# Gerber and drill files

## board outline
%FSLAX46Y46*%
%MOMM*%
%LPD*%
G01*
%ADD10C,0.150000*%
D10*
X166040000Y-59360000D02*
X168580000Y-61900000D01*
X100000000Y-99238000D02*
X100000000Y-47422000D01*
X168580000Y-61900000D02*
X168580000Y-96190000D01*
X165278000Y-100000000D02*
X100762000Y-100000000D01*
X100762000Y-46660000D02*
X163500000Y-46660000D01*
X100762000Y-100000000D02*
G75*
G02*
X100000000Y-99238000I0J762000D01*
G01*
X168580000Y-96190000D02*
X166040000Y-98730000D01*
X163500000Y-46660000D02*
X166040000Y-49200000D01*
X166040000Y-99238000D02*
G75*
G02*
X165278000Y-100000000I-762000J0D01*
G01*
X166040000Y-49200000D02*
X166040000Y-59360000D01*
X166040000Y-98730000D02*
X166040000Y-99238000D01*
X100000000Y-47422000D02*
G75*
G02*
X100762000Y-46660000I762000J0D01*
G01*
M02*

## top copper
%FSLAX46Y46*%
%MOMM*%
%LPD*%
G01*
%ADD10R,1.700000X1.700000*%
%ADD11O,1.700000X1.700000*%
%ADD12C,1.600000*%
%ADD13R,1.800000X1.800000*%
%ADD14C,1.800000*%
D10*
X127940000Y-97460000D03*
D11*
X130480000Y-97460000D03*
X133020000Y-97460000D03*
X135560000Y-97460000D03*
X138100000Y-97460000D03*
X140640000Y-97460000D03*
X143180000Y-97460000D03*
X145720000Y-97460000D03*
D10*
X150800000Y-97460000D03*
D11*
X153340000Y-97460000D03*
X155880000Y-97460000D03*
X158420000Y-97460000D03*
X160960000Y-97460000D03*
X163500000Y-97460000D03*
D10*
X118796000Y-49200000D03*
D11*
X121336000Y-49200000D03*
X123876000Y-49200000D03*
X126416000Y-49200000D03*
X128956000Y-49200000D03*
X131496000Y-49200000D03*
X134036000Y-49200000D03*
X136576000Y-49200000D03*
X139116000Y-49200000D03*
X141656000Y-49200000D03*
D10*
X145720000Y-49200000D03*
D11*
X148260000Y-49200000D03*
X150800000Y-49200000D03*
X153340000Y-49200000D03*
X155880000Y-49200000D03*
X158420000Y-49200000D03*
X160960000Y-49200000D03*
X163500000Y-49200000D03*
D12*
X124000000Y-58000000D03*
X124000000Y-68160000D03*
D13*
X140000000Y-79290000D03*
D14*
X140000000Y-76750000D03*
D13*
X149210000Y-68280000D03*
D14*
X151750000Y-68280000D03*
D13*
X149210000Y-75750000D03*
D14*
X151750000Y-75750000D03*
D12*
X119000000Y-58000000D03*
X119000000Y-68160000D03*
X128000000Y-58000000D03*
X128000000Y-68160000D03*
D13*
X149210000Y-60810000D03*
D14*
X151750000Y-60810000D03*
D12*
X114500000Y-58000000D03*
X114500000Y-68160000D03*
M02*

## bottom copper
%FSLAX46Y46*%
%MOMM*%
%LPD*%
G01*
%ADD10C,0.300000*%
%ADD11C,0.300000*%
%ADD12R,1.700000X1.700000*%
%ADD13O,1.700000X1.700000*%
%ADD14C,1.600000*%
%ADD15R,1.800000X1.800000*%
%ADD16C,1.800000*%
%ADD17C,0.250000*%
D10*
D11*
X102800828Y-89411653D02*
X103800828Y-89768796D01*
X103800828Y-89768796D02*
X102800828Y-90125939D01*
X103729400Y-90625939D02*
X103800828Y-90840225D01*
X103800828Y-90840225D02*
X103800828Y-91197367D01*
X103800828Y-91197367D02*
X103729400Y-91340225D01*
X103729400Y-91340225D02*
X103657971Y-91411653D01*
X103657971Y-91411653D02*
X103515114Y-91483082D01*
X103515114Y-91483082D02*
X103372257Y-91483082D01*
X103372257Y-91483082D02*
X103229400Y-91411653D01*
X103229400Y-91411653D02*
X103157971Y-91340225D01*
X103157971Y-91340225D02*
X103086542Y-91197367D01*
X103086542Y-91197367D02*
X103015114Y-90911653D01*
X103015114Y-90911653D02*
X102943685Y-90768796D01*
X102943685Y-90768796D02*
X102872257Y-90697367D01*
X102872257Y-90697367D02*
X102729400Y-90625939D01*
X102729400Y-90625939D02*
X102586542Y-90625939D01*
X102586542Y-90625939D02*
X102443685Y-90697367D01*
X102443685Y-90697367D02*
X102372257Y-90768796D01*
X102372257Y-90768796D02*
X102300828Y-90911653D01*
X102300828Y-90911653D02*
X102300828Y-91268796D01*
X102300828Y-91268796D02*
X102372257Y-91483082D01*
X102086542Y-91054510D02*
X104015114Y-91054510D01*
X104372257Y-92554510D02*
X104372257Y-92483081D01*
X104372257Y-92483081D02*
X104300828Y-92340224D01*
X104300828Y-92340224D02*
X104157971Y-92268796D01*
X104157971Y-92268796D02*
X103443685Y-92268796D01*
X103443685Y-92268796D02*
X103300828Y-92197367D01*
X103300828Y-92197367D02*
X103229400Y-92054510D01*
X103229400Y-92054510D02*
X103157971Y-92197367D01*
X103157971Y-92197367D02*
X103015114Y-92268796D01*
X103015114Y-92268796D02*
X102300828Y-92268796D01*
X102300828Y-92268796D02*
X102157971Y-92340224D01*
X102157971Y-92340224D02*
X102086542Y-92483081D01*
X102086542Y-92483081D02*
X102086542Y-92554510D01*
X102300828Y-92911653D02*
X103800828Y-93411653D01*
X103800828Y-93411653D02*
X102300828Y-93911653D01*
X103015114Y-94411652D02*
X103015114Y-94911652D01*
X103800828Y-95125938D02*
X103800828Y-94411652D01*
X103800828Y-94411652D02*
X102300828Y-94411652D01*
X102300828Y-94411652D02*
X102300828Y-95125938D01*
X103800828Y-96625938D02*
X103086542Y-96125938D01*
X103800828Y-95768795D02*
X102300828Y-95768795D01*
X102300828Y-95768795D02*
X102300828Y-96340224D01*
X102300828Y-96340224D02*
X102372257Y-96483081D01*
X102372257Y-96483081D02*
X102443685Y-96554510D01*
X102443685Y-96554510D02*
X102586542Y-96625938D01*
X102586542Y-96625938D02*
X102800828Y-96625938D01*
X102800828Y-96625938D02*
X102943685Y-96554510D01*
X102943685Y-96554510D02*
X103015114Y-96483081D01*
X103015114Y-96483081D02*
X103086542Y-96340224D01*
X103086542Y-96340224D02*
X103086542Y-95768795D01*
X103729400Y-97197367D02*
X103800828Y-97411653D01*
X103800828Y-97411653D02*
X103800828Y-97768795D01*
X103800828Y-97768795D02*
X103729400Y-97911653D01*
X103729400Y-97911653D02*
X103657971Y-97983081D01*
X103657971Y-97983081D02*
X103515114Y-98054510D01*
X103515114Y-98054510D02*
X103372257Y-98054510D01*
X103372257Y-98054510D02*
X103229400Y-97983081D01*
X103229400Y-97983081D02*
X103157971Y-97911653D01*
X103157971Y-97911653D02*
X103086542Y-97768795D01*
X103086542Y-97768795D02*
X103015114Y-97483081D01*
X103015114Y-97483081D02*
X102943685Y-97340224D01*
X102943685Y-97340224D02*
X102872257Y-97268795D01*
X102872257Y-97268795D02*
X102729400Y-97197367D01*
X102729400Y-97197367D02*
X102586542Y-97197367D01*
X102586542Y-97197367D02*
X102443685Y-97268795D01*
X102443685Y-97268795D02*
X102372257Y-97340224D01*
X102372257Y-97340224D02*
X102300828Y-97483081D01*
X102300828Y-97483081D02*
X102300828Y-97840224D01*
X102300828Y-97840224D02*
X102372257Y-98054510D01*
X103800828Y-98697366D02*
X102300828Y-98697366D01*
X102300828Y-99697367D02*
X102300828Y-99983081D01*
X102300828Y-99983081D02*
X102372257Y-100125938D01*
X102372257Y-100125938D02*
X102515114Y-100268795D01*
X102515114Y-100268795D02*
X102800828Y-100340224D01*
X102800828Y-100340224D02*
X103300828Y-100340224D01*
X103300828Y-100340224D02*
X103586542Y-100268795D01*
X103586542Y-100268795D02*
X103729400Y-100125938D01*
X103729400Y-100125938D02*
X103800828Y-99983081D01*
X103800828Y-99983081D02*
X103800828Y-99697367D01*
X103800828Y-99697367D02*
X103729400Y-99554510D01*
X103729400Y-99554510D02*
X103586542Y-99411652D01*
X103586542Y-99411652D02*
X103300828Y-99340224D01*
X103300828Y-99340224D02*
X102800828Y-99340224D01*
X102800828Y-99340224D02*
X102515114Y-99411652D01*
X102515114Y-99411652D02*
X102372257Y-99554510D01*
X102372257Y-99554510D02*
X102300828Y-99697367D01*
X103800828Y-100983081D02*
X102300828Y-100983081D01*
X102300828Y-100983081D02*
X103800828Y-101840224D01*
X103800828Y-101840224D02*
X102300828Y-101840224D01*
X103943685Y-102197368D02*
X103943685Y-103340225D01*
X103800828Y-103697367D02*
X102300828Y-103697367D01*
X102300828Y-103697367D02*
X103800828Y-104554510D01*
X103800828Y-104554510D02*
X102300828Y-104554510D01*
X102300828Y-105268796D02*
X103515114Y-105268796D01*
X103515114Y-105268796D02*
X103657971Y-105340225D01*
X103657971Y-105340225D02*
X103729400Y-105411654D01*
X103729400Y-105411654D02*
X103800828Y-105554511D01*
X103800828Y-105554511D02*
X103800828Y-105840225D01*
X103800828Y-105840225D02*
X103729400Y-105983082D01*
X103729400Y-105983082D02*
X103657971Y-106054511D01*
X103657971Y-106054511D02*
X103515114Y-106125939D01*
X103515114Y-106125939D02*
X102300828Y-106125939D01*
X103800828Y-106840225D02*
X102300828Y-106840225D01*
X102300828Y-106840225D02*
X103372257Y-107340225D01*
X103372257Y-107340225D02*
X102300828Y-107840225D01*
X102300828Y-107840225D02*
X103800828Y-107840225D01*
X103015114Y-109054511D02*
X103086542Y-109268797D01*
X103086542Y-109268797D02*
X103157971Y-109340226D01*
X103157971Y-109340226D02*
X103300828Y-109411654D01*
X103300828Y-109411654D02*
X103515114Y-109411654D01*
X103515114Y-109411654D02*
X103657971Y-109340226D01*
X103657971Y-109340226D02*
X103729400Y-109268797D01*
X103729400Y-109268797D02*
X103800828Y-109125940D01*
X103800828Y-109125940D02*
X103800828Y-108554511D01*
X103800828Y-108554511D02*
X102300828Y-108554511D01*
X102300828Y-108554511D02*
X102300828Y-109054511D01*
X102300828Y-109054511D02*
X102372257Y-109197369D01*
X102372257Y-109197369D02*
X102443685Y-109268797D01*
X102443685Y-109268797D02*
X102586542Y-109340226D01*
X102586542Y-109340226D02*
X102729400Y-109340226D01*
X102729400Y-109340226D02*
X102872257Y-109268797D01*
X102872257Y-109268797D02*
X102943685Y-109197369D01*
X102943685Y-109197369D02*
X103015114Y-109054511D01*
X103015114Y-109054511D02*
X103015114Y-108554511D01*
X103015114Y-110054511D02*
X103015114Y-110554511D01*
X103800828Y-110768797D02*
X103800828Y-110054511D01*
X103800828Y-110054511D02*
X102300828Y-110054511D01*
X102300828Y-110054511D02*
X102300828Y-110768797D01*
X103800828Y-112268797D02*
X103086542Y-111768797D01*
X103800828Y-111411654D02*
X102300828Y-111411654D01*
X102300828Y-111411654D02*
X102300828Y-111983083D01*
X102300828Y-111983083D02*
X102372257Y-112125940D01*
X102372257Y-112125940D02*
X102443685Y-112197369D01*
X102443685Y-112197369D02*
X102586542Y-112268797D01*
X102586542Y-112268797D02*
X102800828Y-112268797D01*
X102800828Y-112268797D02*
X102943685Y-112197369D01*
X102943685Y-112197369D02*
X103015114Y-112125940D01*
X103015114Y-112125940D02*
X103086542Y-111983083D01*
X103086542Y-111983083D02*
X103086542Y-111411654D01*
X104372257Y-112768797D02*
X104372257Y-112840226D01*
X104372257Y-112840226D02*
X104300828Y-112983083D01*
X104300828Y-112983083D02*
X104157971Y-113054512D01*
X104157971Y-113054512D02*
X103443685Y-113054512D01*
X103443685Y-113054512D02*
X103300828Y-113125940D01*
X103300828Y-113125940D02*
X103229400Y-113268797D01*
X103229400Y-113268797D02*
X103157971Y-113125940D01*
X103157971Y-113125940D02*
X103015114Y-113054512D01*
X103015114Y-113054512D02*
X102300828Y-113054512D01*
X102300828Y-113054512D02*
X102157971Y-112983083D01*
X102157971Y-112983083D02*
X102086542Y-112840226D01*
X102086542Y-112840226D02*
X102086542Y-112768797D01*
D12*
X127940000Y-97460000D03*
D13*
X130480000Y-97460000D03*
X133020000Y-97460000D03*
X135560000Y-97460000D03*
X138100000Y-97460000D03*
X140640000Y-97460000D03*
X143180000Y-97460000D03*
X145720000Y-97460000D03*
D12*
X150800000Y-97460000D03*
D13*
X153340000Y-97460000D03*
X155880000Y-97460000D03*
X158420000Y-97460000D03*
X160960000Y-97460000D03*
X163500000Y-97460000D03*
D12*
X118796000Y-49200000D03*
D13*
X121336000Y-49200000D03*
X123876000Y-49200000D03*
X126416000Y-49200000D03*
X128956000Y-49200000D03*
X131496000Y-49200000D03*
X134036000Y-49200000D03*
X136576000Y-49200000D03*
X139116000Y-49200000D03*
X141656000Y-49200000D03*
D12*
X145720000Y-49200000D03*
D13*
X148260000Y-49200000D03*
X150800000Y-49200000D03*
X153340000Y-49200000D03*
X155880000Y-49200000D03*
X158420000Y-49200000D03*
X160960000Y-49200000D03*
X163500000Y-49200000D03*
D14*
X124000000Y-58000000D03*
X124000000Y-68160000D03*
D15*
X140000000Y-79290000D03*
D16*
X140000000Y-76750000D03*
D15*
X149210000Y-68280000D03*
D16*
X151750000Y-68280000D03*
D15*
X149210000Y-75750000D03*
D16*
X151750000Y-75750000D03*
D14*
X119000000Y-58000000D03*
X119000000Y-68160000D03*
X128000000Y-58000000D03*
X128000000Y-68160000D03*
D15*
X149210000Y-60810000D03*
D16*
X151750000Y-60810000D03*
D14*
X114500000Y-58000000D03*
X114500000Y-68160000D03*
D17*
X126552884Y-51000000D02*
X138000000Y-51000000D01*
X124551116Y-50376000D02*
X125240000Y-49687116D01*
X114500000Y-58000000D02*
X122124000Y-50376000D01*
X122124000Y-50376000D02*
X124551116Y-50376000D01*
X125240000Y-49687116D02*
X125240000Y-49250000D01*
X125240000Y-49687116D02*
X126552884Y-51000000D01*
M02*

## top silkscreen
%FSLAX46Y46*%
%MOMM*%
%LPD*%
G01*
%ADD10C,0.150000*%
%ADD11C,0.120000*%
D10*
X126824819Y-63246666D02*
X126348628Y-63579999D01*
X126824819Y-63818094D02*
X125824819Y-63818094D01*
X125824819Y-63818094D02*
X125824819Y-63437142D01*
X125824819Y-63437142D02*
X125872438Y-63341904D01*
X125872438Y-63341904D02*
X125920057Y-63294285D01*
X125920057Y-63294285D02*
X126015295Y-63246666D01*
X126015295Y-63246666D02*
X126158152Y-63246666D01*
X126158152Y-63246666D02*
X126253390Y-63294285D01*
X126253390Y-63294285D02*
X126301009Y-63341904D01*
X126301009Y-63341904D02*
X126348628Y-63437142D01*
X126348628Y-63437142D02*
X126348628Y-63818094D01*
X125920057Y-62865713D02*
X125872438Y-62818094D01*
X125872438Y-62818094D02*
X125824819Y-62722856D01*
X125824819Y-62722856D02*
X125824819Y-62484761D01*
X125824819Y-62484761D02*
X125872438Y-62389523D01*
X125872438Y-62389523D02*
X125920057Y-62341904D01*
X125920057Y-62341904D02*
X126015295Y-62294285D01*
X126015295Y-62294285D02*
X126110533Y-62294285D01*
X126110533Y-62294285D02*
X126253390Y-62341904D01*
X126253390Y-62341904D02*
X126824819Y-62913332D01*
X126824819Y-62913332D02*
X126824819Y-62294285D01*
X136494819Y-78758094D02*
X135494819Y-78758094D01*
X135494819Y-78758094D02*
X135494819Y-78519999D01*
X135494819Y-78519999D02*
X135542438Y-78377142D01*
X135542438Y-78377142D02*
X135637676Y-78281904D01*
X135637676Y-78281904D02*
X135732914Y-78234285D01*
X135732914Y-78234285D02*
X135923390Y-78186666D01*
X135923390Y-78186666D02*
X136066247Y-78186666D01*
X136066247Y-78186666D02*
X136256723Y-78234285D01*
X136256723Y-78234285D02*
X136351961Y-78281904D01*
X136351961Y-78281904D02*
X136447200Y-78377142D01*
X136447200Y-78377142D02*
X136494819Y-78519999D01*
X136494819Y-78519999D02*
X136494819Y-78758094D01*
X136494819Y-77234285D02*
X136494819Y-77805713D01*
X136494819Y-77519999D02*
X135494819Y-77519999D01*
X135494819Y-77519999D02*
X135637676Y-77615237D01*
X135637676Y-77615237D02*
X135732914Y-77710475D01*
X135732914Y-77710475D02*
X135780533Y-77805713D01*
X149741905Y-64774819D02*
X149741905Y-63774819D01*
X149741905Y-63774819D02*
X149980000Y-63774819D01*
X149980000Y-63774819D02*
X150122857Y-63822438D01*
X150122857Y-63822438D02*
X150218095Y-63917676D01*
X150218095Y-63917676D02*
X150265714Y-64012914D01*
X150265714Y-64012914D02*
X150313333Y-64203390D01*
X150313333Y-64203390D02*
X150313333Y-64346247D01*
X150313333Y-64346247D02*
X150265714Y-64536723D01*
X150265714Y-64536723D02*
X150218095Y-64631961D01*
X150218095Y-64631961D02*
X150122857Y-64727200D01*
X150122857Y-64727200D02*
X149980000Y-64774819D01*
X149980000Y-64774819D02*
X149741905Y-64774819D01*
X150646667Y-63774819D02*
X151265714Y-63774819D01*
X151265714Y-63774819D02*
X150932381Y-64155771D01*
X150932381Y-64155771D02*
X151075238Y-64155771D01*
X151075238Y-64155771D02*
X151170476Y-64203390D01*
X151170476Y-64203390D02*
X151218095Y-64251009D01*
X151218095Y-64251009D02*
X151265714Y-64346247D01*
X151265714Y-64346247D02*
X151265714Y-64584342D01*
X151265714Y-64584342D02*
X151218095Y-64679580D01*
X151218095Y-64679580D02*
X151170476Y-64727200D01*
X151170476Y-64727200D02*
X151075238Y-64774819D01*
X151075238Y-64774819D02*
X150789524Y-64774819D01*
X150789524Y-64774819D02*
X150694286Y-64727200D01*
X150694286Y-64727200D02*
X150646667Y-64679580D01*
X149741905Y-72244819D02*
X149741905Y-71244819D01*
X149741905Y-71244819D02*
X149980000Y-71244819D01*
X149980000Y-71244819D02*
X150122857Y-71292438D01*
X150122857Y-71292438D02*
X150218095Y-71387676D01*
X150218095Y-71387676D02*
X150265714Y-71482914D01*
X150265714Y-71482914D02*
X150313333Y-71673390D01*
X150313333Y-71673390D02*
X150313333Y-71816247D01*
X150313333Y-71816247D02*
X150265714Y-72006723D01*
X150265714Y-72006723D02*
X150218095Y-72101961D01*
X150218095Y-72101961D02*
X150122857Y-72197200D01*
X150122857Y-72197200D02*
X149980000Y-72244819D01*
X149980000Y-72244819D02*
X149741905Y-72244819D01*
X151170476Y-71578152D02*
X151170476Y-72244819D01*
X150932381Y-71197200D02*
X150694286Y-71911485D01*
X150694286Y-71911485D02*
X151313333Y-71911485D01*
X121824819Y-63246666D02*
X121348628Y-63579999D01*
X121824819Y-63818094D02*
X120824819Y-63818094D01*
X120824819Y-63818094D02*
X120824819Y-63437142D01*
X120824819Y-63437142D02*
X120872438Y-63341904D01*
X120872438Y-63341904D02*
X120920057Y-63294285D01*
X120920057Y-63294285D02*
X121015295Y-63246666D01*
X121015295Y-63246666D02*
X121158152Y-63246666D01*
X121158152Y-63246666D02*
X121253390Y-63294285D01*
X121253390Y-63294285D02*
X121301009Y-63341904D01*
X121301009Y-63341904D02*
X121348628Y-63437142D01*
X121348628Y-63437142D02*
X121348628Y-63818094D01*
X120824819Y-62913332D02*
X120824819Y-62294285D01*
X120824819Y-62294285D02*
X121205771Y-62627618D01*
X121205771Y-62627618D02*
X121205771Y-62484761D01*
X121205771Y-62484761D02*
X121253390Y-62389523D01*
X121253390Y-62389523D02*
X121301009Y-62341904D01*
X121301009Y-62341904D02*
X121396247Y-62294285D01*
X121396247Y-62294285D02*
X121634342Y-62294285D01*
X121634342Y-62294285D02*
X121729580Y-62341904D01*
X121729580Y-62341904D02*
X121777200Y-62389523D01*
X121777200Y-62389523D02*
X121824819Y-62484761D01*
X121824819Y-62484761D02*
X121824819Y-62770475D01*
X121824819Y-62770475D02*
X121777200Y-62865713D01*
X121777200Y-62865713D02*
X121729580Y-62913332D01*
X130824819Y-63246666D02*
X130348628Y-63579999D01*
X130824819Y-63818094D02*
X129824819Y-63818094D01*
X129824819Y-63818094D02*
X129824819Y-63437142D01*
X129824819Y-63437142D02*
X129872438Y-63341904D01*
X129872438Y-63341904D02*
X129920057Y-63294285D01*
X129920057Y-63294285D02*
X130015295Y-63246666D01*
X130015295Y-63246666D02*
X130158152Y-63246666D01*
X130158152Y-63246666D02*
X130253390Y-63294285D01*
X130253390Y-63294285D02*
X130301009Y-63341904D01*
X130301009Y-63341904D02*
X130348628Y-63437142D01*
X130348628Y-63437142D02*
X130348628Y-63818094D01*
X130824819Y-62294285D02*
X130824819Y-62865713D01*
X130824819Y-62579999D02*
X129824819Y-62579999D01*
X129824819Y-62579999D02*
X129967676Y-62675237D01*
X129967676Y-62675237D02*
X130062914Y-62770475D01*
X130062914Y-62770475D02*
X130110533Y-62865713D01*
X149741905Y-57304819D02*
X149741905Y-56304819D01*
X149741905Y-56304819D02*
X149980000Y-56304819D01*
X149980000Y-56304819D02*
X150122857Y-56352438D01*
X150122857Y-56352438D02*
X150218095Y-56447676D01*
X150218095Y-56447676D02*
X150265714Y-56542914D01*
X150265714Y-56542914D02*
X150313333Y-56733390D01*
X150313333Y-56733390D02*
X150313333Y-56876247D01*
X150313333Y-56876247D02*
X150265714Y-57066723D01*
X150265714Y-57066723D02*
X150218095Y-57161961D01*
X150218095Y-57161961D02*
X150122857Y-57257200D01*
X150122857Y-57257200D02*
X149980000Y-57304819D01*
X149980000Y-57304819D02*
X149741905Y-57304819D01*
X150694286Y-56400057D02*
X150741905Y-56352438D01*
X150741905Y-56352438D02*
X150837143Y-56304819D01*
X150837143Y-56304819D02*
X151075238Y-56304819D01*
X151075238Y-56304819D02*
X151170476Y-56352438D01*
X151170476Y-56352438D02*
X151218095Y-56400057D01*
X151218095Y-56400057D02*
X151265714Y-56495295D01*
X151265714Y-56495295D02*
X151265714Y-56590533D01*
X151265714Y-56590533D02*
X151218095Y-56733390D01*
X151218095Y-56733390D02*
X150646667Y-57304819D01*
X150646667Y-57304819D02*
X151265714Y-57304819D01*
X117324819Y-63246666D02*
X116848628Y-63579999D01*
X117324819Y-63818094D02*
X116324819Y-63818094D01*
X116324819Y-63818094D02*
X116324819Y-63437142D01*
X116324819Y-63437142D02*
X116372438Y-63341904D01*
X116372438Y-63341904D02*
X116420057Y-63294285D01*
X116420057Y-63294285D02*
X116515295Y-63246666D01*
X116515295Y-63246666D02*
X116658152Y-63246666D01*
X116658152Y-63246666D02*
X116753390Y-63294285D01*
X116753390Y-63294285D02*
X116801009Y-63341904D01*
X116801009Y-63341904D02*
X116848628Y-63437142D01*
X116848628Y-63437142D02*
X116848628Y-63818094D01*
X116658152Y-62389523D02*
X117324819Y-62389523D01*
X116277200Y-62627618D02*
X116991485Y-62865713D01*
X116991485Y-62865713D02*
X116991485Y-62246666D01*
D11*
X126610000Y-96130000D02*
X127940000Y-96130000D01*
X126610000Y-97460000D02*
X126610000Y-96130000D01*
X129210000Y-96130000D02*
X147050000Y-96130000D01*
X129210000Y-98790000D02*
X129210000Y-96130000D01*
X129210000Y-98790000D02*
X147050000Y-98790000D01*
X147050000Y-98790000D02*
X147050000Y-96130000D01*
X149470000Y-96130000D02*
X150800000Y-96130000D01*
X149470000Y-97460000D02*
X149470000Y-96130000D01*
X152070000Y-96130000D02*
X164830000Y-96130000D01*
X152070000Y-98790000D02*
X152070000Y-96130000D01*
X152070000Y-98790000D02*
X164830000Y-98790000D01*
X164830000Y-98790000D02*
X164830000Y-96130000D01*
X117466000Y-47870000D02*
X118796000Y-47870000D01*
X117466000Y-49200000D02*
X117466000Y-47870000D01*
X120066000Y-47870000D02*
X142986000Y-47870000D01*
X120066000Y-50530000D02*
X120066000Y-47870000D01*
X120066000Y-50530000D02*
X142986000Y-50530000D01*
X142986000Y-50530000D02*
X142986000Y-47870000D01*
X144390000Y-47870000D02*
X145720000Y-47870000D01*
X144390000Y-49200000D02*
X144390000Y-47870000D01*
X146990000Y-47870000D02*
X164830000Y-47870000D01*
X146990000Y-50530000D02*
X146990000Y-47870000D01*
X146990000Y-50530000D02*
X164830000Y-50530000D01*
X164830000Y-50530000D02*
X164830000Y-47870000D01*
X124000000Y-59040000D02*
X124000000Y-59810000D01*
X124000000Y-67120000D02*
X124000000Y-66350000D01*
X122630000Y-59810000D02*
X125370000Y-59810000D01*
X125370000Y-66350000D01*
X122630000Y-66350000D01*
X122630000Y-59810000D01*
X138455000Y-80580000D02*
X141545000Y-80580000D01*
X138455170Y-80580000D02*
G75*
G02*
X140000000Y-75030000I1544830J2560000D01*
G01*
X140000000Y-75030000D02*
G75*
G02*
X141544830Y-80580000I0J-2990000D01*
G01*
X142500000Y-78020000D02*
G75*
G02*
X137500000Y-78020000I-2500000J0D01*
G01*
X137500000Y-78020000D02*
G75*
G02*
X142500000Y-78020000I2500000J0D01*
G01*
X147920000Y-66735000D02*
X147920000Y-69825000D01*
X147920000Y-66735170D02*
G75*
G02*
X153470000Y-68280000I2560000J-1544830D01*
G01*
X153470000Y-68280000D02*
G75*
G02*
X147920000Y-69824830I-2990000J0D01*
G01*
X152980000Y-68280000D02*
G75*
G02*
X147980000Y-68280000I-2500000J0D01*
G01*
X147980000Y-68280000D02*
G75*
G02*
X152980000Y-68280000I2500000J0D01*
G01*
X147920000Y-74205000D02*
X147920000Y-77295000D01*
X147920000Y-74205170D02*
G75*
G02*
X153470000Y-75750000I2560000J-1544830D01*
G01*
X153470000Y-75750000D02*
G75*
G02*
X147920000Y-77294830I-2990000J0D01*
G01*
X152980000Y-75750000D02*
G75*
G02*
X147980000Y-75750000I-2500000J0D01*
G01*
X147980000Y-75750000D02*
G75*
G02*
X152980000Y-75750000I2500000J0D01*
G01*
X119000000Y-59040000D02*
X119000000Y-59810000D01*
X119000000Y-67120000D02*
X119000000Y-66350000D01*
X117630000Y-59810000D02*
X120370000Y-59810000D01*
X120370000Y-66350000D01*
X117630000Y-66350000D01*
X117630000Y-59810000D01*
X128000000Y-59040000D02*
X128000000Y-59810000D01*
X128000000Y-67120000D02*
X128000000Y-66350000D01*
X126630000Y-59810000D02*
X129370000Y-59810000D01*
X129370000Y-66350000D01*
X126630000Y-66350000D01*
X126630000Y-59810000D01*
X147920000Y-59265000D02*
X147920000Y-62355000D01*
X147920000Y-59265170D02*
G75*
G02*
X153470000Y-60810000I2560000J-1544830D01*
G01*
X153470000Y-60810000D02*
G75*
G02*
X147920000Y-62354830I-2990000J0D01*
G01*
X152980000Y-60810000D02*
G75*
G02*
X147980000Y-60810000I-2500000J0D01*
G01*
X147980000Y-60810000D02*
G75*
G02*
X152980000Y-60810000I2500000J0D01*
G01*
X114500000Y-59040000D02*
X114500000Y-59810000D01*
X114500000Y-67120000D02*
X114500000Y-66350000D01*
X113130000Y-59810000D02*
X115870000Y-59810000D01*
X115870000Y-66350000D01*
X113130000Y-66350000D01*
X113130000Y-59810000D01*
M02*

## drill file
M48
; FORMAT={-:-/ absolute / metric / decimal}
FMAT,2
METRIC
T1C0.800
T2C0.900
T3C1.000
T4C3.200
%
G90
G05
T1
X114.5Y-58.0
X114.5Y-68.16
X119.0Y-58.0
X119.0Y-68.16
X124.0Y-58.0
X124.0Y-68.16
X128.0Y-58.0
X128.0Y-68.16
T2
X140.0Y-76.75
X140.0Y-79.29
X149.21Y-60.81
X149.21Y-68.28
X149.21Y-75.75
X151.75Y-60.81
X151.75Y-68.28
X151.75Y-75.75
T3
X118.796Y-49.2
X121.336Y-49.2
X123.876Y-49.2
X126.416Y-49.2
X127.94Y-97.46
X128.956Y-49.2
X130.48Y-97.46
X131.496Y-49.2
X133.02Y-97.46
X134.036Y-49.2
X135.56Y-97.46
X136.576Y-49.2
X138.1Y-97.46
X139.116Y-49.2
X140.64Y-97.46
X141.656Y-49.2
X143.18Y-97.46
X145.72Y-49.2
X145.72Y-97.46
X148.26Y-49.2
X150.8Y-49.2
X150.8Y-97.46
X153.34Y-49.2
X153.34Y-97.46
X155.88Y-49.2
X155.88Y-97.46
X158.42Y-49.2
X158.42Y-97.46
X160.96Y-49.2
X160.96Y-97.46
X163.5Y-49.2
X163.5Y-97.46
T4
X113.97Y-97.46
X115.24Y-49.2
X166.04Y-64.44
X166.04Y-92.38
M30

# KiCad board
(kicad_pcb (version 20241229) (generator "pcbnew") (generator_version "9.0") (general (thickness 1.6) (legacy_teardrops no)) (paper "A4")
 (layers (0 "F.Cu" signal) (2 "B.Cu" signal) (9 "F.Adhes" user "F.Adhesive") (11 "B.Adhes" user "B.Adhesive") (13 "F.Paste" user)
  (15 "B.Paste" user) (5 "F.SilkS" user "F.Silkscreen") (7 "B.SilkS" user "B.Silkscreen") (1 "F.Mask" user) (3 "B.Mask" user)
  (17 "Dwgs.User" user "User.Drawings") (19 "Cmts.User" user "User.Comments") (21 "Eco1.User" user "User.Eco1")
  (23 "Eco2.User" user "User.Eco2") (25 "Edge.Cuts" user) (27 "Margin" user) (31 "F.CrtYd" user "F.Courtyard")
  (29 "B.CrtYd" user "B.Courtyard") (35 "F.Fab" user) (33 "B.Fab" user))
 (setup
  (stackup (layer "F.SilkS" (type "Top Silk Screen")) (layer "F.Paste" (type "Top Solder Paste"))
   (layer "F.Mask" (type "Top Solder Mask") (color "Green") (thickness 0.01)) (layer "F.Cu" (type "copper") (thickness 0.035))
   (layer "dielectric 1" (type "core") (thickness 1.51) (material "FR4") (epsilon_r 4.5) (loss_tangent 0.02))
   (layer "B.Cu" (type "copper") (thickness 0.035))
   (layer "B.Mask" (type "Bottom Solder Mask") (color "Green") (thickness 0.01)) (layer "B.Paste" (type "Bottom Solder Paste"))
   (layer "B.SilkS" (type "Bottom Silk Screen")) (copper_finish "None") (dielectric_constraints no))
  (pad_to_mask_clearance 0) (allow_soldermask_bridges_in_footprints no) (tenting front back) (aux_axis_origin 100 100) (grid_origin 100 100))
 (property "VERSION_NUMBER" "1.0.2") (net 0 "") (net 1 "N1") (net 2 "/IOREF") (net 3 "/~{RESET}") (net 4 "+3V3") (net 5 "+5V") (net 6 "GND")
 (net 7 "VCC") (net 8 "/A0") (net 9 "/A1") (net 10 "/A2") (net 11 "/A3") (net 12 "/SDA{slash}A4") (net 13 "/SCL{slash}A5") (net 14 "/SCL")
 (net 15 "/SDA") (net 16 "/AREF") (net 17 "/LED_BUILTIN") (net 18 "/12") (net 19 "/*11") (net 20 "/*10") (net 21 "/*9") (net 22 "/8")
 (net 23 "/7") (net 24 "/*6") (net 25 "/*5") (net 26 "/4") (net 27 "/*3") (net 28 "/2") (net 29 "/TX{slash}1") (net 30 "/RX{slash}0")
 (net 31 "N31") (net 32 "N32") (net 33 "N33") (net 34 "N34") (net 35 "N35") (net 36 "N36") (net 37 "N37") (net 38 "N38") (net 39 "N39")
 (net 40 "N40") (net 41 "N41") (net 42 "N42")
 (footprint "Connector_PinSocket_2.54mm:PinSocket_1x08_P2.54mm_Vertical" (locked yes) (layer "F.Cu") (at 127.94 97.46 90)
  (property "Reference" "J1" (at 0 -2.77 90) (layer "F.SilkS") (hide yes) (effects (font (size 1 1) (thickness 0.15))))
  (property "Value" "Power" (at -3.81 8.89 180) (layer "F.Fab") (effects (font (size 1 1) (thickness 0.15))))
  (fp_line (start 1.33 -1.33) (end 1.33 0) (stroke (width 0.12) (type solid)) (layer "F.SilkS"))
  (fp_line (start 0 -1.33) (end 1.33 -1.33) (stroke (width 0.12) (type solid)) (layer "F.SilkS"))
  (fp_line (start 1.33 1.27) (end 1.33 19.11) (stroke (width 0.12) (type solid)) (layer "F.SilkS"))
  (fp_line (start -1.33 1.27) (end 1.33 1.27) (stroke (width 0.12) (type solid)) (layer "F.SilkS"))
  (fp_line (start -1.33 1.27) (end -1.33 19.11) (stroke (width 0.12) (type solid)) (layer "F.SilkS"))
  (fp_line (start -1.33 19.11) (end 1.33 19.11) (stroke (width 0.12) (type solid)) (layer "F.SilkS"))
  (pad "1" thru_hole rect (at 0 0 90) (size 1.7 1.7) (drill 1) (layers "*.Cu" "*.Mask") (remove_unused_layers no) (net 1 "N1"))
  (pad "2" thru_hole oval (at 0 2.54 90) (size 1.7 1.7) (drill 1) (layers "*.Cu" "*.Mask") (remove_unused_layers no) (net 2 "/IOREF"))
  (pad "3" thru_hole oval (at 0 5.08 90) (size 1.7 1.7) (drill 1) (layers "*.Cu" "*.Mask") (remove_unused_layers no) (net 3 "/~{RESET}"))
  (pad "4" thru_hole oval (at 0 7.62 90) (size 1.7 1.7) (drill 1) (layers "*.Cu" "*.Mask") (remove_unused_layers no) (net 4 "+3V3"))
  (pad "5" thru_hole oval (at 0 10.16 90) (size 1.7 1.7) (drill 1) (layers "*.Cu" "*.Mask") (remove_unused_layers no) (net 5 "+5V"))
  (pad "6" thru_hole oval (at 0 12.7 90) (size 1.7 1.7) (drill 1) (layers "*.Cu" "*.Mask") (remove_unused_layers no) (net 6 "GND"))
  (pad "7" thru_hole oval (at 0 15.24 90) (size 1.7 1.7) (drill 1) (layers "*.Cu" "*.Mask") (remove_unused_layers no) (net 6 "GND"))
  (pad "8" thru_hole oval (at 0 17.78 90) (size 1.7 1.7) (drill 1) (layers "*.Cu" "*.Mask") (remove_unused_layers no) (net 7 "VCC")))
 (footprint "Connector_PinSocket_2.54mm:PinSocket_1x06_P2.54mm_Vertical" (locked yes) (layer "F.Cu") (at 150.8 97.46 90)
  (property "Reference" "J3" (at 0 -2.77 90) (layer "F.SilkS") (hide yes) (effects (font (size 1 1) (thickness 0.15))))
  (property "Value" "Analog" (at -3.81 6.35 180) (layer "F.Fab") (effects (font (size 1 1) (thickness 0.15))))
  (fp_line (start 1.33 -1.33) (end 1.33 0) (stroke (width 0.12) (type solid)) (layer "F.SilkS"))
  (fp_line (start 0 -1.33) (end 1.33 -1.33) (stroke (width 0.12) (type solid)) (layer "F.SilkS"))
  (fp_line (start 1.33 1.27) (end 1.33 14.03) (stroke (width 0.12) (type solid)) (layer "F.SilkS"))
  (fp_line (start -1.33 1.27) (end 1.33 1.27) (stroke (width 0.12) (type solid)) (layer "F.SilkS"))
  (fp_line (start -1.33 1.27) (end -1.33 14.03) (stroke (width 0.12) (type solid)) (layer "F.SilkS"))
  (fp_line (start -1.33 14.03) (end 1.33 14.03) (stroke (width 0.12) (type solid)) (layer "F.SilkS"))
  (pad "1" thru_hole rect (at 0 0 90) (size 1.7 1.7) (drill 1) (layers "*.Cu" "*.Mask") (remove_unused_layers no) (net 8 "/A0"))
  (pad "2" thru_hole oval (at 0 2.54 90) (size 1.7 1.7) (drill 1) (layers "*.Cu" "*.Mask") (remove_unused_layers no) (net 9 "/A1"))
  (pad "3" thru_hole oval (at 0 5.08 90) (size 1.7 1.7) (drill 1) (layers "*.Cu" "*.Mask") (remove_unused_layers no) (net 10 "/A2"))
  (pad "4" thru_hole oval (at 0 7.62 90) (size 1.7 1.7) (drill 1) (layers "*.Cu" "*.Mask") (remove_unused_layers no) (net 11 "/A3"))
  (pad "5" thru_hole oval (at 0 10.16 90) (size 1.7 1.7) (drill 1) (layers "*.Cu" "*.Mask") (remove_unused_layers no)
   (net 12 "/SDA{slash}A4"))
  (pad "6" thru_hole oval (at 0 12.7 90) (size 1.7 1.7) (drill 1) (layers "*.Cu" "*.Mask") (remove_unused_layers no)
   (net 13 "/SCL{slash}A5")))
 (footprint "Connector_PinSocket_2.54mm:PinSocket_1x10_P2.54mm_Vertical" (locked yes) (layer "F.Cu") (at 118.796 49.2 90)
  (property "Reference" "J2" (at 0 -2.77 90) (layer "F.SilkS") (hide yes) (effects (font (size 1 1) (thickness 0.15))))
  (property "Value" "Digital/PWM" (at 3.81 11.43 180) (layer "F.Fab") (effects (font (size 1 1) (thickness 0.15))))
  (fp_line (start 1.33 -1.33) (end 1.33 0) (stroke (width 0.12) (type solid)) (layer "F.SilkS"))
  (fp_line (start 0 -1.33) (end 1.33 -1.33) (stroke (width 0.12) (type solid)) (layer "F.SilkS"))
  (fp_line (start 1.33 1.27) (end 1.33 24.19) (stroke (width 0.12) (type solid)) (layer "F.SilkS"))
  (fp_line (start -1.33 1.27) (end 1.33 1.27) (stroke (width 0.12) (type solid)) (layer "F.SilkS"))
  (fp_line (start -1.33 1.27) (end -1.33 24.19) (stroke (width 0.12) (type solid)) (layer "F.SilkS"))
  (fp_line (start -1.33 24.19) (end 1.33 24.19) (stroke (width 0.12) (type solid)) (layer "F.SilkS"))
  (pad "1" thru_hole rect (at 0 0 90) (size 1.7 1.7) (drill 1) (layers "*.Cu" "*.Mask") (remove_unused_layers no) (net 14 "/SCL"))
  (pad "2" thru_hole oval (at 0 2.54 90) (size 1.7 1.7) (drill 1) (layers "*.Cu" "*.Mask") (remove_unused_layers no) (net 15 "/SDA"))
  (pad "3" thru_hole oval (at 0 5.08 90) (size 1.7 1.7) (drill 1) (layers "*.Cu" "*.Mask") (remove_unused_layers no) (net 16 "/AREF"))
  (pad "4" thru_hole oval (at 0 7.62 90) (size 1.7 1.7) (drill 1) (layers "*.Cu" "*.Mask") (remove_unused_layers no) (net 6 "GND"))
  (pad "5" thru_hole oval (at 0 10.16 90) (size 1.7 1.7) (drill 1) (layers "*.Cu" "*.Mask") (remove_unused_layers no)
   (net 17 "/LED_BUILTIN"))
  (pad "6" thru_hole oval (at 0 12.7 90) (size 1.7 1.7) (drill 1) (layers "*.Cu" "*.Mask") (remove_unused_layers no) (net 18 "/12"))
  (pad "7" thru_hole oval (at 0 15.24 90) (size 1.7 1.7) (drill 1) (layers "*.Cu" "*.Mask") (remove_unused_layers no) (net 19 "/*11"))
  (pad "8" thru_hole oval (at 0 17.78 90) (size 1.7 1.7) (drill 1) (layers "*.Cu" "*.Mask") (remove_unused_layers no) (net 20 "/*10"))
  (pad "9" thru_hole oval (at 0 20.32 90) (size 1.7 1.7) (drill 1) (layers "*.Cu" "*.Mask") (remove_unused_layers no) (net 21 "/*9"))
  (pad "10" thru_hole oval (at 0 22.86 90) (size 1.7 1.7) (drill 1) (layers "*.Cu" "*.Mask") (remove_unused_layers no) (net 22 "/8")))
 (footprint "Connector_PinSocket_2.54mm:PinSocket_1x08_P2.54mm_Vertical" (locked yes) (layer "F.Cu") (at 145.72 49.2 90)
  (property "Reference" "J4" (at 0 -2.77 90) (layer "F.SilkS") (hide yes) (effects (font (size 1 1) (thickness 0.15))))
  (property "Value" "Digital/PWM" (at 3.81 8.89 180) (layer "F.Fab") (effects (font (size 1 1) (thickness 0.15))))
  (fp_line (start 1.33 -1.33) (end 1.33 0) (stroke (width 0.12) (type solid)) (layer "F.SilkS"))
  (fp_line (start 0 -1.33) (end 1.33 -1.33) (stroke (width 0.12) (type solid)) (layer "F.SilkS"))
  (fp_line (start 1.33 1.27) (end 1.33 19.11) (stroke (width 0.12) (type solid)) (layer "F.SilkS"))
  (fp_line (start -1.33 1.27) (end 1.33 1.27) (stroke (width 0.12) (type solid)) (layer "F.SilkS"))
  (fp_line (start -1.33 1.27) (end -1.33 19.11) (stroke (width 0.12) (type solid)) (layer "F.SilkS"))
  (fp_line (start -1.33 19.11) (end 1.33 19.11) (stroke (width 0.12) (type solid)) (layer "F.SilkS"))
  (pad "1" thru_hole rect (at 0 0 90) (size 1.7 1.7) (drill 1) (layers "*.Cu" "*.Mask") (remove_unused_layers no) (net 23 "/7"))
  (pad "2" thru_hole oval (at 0 2.54 90) (size 1.7 1.7) (drill 1) (layers "*.Cu" "*.Mask") (remove_unused_layers no) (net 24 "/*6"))
  (pad "3" thru_hole oval (at 0 5.08 90) (size 1.7 1.7) (drill 1) (layers "*.Cu" "*.Mask") (remove_unused_layers no) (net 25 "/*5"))
  (pad "4" thru_hole oval (at 0 7.62 90) (size 1.7 1.7) (drill 1) (layers "*.Cu" "*.Mask") (remove_unused_layers no) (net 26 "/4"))
  (pad "5" thru_hole oval (at 0 10.16 90) (size 1.7 1.7) (drill 1) (layers "*.Cu" "*.Mask") (remove_unused_layers no) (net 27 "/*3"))
  (pad "6" thru_hole oval (at 0 12.7 90) (size 1.7 1.7) (drill 1) (layers "*.Cu" "*.Mask") (remove_unused_layers no) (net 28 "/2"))
  (pad "7" thru_hole oval (at 0 15.24 90) (size 1.7 1.7) (drill 1) (layers "*.Cu" "*.Mask") (remove_unused_layers no) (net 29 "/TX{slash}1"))
  (pad "8" thru_hole oval (at 0 17.78 90) (size 1.7 1.7) (drill 1) (layers "*.Cu" "*.Mask") (remove_unused_layers no) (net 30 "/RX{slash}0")))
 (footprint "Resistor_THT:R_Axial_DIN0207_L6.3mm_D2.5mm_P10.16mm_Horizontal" (layer "F.Cu") (at 124 58 -90)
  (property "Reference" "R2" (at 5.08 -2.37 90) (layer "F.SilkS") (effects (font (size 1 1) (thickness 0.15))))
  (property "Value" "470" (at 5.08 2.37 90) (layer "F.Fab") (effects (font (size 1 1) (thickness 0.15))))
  (fp_line (start 1.04 0) (end 1.81 0) (stroke (width 0.12) (type solid)) (layer "F.SilkS"))
  (fp_line (start 9.12 0) (end 8.35 0) (stroke (width 0.12) (type solid)) (layer "F.SilkS"))
  (fp_rect (start 1.81 -1.37) (end 8.35 1.37) (stroke (width 0.12) (type solid)) (fill no) (layer "F.SilkS"))
  (pad "1" thru_hole circle (at 0 0 270) (size 1.6 1.6) (drill 0.8) (layers "*.Cu" "*.Mask") (remove_unused_layers no) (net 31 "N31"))
  (pad "2" thru_hole circle (at 10.16 0 270) (size 1.6 1.6) (drill 0.8) (layers "*.Cu" "*.Mask") (remove_unused_layers no) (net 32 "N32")))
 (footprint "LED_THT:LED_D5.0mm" (layer "F.Cu") (at 140 79.29 90)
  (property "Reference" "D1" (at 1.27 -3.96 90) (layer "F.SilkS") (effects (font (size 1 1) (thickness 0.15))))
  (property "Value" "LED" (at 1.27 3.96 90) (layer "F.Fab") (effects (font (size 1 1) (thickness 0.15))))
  (fp_line (start -1.29 -1.545) (end -1.29 1.545) (stroke (width 0.12) (type solid)) (layer "F.SilkS"))
  (fp_arc (start -1.29 -1.54483) (mid 2.071779 -2.880495) (end 4.26 0) (stroke (width 0.12) (type solid)) (layer "F.SilkS"))
  (fp_arc (start 4.26 0) (mid 2.071779 2.880495) (end -1.29 1.54483) (stroke (width 0.12) (type solid)) (layer "F.SilkS"))
  (fp_circle (center 1.27 0) (end 3.77 0) (stroke (width 0.12) (type solid)) (fill no) (layer "F.SilkS"))
  (pad "1" thru_hole rect (at 0 0 90) (size 1.8 1.8) (drill 0.9) (layers "*.Cu" "*.Mask") (remove_unused_layers no) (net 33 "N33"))
  (pad "2" thru_hole circle (at 2.54 0 90) (size 1.8 1.8) (drill 0.9) (layers "*.Cu" "*.Mask") (remove_unused_layers no) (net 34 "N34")))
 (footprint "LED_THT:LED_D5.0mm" (layer "F.Cu") (at 149.21 68.28)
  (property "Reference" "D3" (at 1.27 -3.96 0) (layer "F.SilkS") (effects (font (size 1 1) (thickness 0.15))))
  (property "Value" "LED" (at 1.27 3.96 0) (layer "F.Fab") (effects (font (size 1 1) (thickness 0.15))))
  (fp_line (start -1.29 -1.545) (end -1.29 1.545) (stroke (width 0.12) (type solid)) (layer "F.SilkS"))
  (fp_arc (start -1.29 -1.54483) (mid 2.071779 -2.880495) (end 4.26 0) (stroke (width 0.12) (type solid)) (layer "F.SilkS"))
  (fp_arc (start 4.26 0) (mid 2.071779 2.880495) (end -1.29 1.54483) (stroke (width 0.12) (type solid)) (layer "F.SilkS"))
  (fp_circle (center 1.27 0) (end 3.77 0) (stroke (width 0.12) (type solid)) (fill no) (layer "F.SilkS"))
  (pad "1" thru_hole rect (at 0 0) (size 1.8 1.8) (drill 0.9) (layers "*.Cu" "*.Mask") (remove_unused_layers no) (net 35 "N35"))
  (pad "2" thru_hole circle (at 2.54 0) (size 1.8 1.8) (drill 0.9) (layers "*.Cu" "*.Mask") (remove_unused_layers no) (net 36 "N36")))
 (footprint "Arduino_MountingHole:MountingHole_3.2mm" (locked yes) (layer "F.Cu") (at 115.24 49.2)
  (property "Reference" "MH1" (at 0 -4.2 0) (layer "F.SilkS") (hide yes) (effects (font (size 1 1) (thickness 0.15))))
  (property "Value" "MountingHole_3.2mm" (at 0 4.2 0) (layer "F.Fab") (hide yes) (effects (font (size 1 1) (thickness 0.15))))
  (pad "" np_thru_hole circle (at 0 0) (size 3.2 3.2) (drill 3.2) (layers "*.Cu" "*.Mask")))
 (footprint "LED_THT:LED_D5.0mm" (layer "F.Cu") (at 149.21 75.75)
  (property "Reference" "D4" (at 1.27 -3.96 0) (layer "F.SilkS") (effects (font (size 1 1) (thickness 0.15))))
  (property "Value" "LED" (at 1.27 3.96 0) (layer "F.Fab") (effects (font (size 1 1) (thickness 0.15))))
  (fp_line (start -1.29 -1.545) (end -1.29 1.545) (stroke (width 0.12) (type solid)) (layer "F.SilkS"))
  (fp_arc (start -1.29 -1.54483) (mid 2.071779 -2.880495) (end 4.26 0) (stroke (width 0.12) (type solid)) (layer "F.SilkS"))
  (fp_arc (start 4.26 0) (mid 2.071779 2.880495) (end -1.29 1.54483) (stroke (width 0.12) (type solid)) (layer "F.SilkS"))
  (fp_circle (center 1.27 0) (end 3.77 0) (stroke (width 0.12) (type solid)) (fill no) (layer "F.SilkS"))
  (pad "1" thru_hole rect (at 0 0) (size 1.8 1.8) (drill 0.9) (layers "*.Cu" "*.Mask") (remove_unused_layers no) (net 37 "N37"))
  (pad "2" thru_hole circle (at 2.54 0) (size 1.8 1.8) (drill 0.9) (layers "*.Cu" "*.Mask") (remove_unused_layers no) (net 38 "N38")))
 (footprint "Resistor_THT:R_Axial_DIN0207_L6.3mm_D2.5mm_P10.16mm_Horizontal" (layer "F.Cu") (at 119 58 -90)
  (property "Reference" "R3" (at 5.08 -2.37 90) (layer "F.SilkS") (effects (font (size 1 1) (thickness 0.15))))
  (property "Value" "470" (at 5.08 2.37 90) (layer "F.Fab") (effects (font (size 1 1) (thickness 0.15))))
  (fp_line (start 1.04 0) (end 1.81 0) (stroke (width 0.12) (type solid)) (layer "F.SilkS"))
  (fp_line (start 9.12 0) (end 8.35 0) (stroke (width 0.12) (type solid)) (layer "F.SilkS"))
  (fp_rect (start 1.81 -1.37) (end 8.35 1.37) (stroke (width 0.12) (type solid)) (fill no) (layer "F.SilkS"))
  (pad "1" thru_hole circle (at 0 0 270) (size 1.6 1.6) (drill 0.8) (layers "*.Cu" "*.Mask") (remove_unused_layers no) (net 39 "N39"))
  (pad "2" thru_hole circle (at 10.16 0 270) (size 1.6 1.6) (drill 0.8) (layers "*.Cu" "*.Mask") (remove_unused_layers no) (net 36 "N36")))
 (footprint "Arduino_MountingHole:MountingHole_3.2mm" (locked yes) (layer "F.Cu") (at 113.97 97.46)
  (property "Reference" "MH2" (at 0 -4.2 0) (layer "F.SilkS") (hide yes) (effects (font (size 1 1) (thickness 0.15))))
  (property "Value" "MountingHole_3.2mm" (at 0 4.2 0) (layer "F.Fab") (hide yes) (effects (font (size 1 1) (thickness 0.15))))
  (pad "" np_thru_hole circle (at 0 0) (size 3.2 3.2) (drill 3.2) (layers "*.Cu" "*.Mask")))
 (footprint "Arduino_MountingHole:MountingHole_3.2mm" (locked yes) (layer "F.Cu") (at 166.04 64.44)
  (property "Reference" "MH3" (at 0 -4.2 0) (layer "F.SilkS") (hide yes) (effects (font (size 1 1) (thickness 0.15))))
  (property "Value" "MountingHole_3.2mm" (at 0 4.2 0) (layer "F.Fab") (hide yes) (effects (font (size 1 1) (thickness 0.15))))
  (pad "" np_thru_hole circle (at 0 0) (size 3.2 3.2) (drill 3.2) (layers "*.Cu" "*.Mask")))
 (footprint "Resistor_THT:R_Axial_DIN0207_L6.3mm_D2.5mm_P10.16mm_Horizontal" (layer "F.Cu") (at 128 58 -90)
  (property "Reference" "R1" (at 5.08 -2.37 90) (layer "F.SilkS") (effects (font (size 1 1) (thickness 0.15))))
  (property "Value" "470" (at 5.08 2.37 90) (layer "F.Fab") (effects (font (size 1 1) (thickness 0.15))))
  (fp_line (start 1.04 0) (end 1.81 0) (stroke (width 0.12) (type solid)) (layer "F.SilkS"))
  (fp_line (start 9.12 0) (end 8.35 0) (stroke (width 0.12) (type solid)) (layer "F.SilkS"))
  (fp_rect (start 1.81 -1.37) (end 8.35 1.37) (stroke (width 0.12) (type solid)) (fill no) (layer "F.SilkS"))
  (pad "1" thru_hole circle (at 0 0 270) (size 1.6 1.6) (drill 0.8) (layers "*.Cu" "*.Mask") (remove_unused_layers no) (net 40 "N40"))
  (pad "2" thru_hole circle (at 10.16 0 270) (size 1.6 1.6) (drill 0.8) (layers "*.Cu" "*.Mask") (remove_unused_layers no) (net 34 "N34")))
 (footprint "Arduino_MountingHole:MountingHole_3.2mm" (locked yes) (layer "F.Cu") (at 166.04 92.38)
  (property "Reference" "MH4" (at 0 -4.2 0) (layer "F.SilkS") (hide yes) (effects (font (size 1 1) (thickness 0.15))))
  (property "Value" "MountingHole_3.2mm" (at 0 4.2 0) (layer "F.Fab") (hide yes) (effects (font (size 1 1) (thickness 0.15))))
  (pad "" np_thru_hole circle (at 0 0) (size 3.2 3.2) (drill 3.2) (layers "*.Cu" "*.Mask")))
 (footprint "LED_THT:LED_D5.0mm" (layer "F.Cu") (at 149.21 60.81)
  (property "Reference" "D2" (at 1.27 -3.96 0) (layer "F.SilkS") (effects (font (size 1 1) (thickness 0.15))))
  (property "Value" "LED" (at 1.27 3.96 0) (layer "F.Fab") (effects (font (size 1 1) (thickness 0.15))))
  (fp_line (start -1.29 -1.545) (end -1.29 1.545) (stroke (width 0.12) (type solid)) (layer "F.SilkS"))
  (fp_arc (start -1.29 -1.54483) (mid 2.071779 -2.880495) (end 4.26 0) (stroke (width 0.12) (type solid)) (layer "F.SilkS"))
  (fp_arc (start 4.26 0) (mid 2.071779 2.880495) (end -1.29 1.54483) (stroke (width 0.12) (type solid)) (layer "F.SilkS"))
  (fp_circle (center 1.27 0) (end 3.77 0) (stroke (width 0.12) (type solid)) (fill no) (layer "F.SilkS"))
  (pad "1" thru_hole rect (at 0 0) (size 1.8 1.8) (drill 0.9) (layers "*.Cu" "*.Mask") (remove_unused_layers no) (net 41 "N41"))
  (pad "2" thru_hole circle (at 2.54 0) (size 1.8 1.8) (drill 0.9) (layers "*.Cu" "*.Mask") (remove_unused_layers no) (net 32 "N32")))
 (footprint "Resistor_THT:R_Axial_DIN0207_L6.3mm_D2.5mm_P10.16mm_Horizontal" (layer "F.Cu") (at 114.5 58 -90)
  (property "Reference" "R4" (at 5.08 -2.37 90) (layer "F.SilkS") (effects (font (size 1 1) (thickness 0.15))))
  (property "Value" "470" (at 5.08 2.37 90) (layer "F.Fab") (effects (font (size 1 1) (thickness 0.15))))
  (fp_line (start 1.04 0) (end 1.81 0) (stroke (width 0.12) (type solid)) (layer "F.SilkS"))
  (fp_line (start 9.12 0) (end 8.35 0) (stroke (width 0.12) (type solid)) (layer "F.SilkS"))
  (fp_rect (start 1.81 -1.37) (end 8.35 1.37) (stroke (width 0.12) (type solid)) (fill no) (layer "F.SilkS"))
  (pad "1" thru_hole circle (at 0 0 270) (size 1.6 1.6) (drill 0.8) (layers "*.Cu" "*.Mask") (remove_unused_layers no) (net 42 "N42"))
  (pad "2" thru_hole circle (at 10.16 0 270) (size 1.6 1.6) (drill 0.8) (layers "*.Cu" "*.Mask") (remove_unused_layers no) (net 38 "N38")))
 (gr_line (start 166.04 59.36) (end 168.58 61.9) (stroke (width 0.15) (type solid)) (layer "Edge.Cuts"))
 (gr_line (start 100 99.238) (end 100 47.422) (stroke (width 0.15) (type solid)) (layer "Edge.Cuts"))
 (gr_line (start 168.58 61.9) (end 168.58 96.19) (stroke (width 0.15) (type solid)) (layer "Edge.Cuts"))
 (gr_line (start 165.278 100) (end 100.762 100) (stroke (width 0.15) (type solid)) (layer "Edge.Cuts"))
 (gr_line (start 100.762 46.66) (end 163.5 46.66) (stroke (width 0.15) (type solid)) (layer "Edge.Cuts"))
 (gr_arc (start 100.762 100) (mid 100.223185 99.776815) (end 100 99.238) (stroke (width 0.15) (type solid)) (layer "Edge.Cuts"))
 (gr_line (start 168.58 96.19) (end 166.04 98.73) (stroke (width 0.15) (type solid)) (layer "Edge.Cuts"))
 (gr_line (start 163.5 46.66) (end 166.04 49.2) (stroke (width 0.15) (type solid)) (layer "Edge.Cuts"))
 (gr_arc (start 166.04 99.238) (mid 165.816815 99.776815) (end 165.278 100) (stroke (width 0.15) (type solid)) (layer "Edge.Cuts"))
 (gr_line (start 166.04 49.2) (end 166.04 59.36) (stroke (width 0.15) (type solid)) (layer "Edge.Cuts"))
 (gr_line (start 166.04 98.73) (end 166.04 99.238) (stroke (width 0.15) (type solid)) (layer "Edge.Cuts"))
 (gr_arc (start 100 47.422) (mid 100.223185 46.883185) (end 100.762 46.66) (stroke (width 0.15) (type solid)) (layer "Edge.Cuts"))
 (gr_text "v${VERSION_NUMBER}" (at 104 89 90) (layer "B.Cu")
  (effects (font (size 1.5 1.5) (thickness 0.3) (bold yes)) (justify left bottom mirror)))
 (segment (start 126.552884 51) (end 138 51) (width 0.25) (layer "B.Cu") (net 42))
 (segment (start 124.551116 50.376) (end 125.24 49.687116) (width 0.25) (layer "B.Cu") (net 42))
 (segment (start 114.5 58) (end 122.124 50.376) (width 0.25) (layer "B.Cu") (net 42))
 (segment (start 122.124 50.376) (end 124.551116 50.376) (width 0.25) (layer "B.Cu") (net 42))
 (segment (start 125.24 49.687116) (end 125.24 49.25) (width 0.25) (layer "B.Cu") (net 42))
 (segment (start 125.24 49.687116) (end 126.552884 51) (width 0.25) (layer "B.Cu") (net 42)))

